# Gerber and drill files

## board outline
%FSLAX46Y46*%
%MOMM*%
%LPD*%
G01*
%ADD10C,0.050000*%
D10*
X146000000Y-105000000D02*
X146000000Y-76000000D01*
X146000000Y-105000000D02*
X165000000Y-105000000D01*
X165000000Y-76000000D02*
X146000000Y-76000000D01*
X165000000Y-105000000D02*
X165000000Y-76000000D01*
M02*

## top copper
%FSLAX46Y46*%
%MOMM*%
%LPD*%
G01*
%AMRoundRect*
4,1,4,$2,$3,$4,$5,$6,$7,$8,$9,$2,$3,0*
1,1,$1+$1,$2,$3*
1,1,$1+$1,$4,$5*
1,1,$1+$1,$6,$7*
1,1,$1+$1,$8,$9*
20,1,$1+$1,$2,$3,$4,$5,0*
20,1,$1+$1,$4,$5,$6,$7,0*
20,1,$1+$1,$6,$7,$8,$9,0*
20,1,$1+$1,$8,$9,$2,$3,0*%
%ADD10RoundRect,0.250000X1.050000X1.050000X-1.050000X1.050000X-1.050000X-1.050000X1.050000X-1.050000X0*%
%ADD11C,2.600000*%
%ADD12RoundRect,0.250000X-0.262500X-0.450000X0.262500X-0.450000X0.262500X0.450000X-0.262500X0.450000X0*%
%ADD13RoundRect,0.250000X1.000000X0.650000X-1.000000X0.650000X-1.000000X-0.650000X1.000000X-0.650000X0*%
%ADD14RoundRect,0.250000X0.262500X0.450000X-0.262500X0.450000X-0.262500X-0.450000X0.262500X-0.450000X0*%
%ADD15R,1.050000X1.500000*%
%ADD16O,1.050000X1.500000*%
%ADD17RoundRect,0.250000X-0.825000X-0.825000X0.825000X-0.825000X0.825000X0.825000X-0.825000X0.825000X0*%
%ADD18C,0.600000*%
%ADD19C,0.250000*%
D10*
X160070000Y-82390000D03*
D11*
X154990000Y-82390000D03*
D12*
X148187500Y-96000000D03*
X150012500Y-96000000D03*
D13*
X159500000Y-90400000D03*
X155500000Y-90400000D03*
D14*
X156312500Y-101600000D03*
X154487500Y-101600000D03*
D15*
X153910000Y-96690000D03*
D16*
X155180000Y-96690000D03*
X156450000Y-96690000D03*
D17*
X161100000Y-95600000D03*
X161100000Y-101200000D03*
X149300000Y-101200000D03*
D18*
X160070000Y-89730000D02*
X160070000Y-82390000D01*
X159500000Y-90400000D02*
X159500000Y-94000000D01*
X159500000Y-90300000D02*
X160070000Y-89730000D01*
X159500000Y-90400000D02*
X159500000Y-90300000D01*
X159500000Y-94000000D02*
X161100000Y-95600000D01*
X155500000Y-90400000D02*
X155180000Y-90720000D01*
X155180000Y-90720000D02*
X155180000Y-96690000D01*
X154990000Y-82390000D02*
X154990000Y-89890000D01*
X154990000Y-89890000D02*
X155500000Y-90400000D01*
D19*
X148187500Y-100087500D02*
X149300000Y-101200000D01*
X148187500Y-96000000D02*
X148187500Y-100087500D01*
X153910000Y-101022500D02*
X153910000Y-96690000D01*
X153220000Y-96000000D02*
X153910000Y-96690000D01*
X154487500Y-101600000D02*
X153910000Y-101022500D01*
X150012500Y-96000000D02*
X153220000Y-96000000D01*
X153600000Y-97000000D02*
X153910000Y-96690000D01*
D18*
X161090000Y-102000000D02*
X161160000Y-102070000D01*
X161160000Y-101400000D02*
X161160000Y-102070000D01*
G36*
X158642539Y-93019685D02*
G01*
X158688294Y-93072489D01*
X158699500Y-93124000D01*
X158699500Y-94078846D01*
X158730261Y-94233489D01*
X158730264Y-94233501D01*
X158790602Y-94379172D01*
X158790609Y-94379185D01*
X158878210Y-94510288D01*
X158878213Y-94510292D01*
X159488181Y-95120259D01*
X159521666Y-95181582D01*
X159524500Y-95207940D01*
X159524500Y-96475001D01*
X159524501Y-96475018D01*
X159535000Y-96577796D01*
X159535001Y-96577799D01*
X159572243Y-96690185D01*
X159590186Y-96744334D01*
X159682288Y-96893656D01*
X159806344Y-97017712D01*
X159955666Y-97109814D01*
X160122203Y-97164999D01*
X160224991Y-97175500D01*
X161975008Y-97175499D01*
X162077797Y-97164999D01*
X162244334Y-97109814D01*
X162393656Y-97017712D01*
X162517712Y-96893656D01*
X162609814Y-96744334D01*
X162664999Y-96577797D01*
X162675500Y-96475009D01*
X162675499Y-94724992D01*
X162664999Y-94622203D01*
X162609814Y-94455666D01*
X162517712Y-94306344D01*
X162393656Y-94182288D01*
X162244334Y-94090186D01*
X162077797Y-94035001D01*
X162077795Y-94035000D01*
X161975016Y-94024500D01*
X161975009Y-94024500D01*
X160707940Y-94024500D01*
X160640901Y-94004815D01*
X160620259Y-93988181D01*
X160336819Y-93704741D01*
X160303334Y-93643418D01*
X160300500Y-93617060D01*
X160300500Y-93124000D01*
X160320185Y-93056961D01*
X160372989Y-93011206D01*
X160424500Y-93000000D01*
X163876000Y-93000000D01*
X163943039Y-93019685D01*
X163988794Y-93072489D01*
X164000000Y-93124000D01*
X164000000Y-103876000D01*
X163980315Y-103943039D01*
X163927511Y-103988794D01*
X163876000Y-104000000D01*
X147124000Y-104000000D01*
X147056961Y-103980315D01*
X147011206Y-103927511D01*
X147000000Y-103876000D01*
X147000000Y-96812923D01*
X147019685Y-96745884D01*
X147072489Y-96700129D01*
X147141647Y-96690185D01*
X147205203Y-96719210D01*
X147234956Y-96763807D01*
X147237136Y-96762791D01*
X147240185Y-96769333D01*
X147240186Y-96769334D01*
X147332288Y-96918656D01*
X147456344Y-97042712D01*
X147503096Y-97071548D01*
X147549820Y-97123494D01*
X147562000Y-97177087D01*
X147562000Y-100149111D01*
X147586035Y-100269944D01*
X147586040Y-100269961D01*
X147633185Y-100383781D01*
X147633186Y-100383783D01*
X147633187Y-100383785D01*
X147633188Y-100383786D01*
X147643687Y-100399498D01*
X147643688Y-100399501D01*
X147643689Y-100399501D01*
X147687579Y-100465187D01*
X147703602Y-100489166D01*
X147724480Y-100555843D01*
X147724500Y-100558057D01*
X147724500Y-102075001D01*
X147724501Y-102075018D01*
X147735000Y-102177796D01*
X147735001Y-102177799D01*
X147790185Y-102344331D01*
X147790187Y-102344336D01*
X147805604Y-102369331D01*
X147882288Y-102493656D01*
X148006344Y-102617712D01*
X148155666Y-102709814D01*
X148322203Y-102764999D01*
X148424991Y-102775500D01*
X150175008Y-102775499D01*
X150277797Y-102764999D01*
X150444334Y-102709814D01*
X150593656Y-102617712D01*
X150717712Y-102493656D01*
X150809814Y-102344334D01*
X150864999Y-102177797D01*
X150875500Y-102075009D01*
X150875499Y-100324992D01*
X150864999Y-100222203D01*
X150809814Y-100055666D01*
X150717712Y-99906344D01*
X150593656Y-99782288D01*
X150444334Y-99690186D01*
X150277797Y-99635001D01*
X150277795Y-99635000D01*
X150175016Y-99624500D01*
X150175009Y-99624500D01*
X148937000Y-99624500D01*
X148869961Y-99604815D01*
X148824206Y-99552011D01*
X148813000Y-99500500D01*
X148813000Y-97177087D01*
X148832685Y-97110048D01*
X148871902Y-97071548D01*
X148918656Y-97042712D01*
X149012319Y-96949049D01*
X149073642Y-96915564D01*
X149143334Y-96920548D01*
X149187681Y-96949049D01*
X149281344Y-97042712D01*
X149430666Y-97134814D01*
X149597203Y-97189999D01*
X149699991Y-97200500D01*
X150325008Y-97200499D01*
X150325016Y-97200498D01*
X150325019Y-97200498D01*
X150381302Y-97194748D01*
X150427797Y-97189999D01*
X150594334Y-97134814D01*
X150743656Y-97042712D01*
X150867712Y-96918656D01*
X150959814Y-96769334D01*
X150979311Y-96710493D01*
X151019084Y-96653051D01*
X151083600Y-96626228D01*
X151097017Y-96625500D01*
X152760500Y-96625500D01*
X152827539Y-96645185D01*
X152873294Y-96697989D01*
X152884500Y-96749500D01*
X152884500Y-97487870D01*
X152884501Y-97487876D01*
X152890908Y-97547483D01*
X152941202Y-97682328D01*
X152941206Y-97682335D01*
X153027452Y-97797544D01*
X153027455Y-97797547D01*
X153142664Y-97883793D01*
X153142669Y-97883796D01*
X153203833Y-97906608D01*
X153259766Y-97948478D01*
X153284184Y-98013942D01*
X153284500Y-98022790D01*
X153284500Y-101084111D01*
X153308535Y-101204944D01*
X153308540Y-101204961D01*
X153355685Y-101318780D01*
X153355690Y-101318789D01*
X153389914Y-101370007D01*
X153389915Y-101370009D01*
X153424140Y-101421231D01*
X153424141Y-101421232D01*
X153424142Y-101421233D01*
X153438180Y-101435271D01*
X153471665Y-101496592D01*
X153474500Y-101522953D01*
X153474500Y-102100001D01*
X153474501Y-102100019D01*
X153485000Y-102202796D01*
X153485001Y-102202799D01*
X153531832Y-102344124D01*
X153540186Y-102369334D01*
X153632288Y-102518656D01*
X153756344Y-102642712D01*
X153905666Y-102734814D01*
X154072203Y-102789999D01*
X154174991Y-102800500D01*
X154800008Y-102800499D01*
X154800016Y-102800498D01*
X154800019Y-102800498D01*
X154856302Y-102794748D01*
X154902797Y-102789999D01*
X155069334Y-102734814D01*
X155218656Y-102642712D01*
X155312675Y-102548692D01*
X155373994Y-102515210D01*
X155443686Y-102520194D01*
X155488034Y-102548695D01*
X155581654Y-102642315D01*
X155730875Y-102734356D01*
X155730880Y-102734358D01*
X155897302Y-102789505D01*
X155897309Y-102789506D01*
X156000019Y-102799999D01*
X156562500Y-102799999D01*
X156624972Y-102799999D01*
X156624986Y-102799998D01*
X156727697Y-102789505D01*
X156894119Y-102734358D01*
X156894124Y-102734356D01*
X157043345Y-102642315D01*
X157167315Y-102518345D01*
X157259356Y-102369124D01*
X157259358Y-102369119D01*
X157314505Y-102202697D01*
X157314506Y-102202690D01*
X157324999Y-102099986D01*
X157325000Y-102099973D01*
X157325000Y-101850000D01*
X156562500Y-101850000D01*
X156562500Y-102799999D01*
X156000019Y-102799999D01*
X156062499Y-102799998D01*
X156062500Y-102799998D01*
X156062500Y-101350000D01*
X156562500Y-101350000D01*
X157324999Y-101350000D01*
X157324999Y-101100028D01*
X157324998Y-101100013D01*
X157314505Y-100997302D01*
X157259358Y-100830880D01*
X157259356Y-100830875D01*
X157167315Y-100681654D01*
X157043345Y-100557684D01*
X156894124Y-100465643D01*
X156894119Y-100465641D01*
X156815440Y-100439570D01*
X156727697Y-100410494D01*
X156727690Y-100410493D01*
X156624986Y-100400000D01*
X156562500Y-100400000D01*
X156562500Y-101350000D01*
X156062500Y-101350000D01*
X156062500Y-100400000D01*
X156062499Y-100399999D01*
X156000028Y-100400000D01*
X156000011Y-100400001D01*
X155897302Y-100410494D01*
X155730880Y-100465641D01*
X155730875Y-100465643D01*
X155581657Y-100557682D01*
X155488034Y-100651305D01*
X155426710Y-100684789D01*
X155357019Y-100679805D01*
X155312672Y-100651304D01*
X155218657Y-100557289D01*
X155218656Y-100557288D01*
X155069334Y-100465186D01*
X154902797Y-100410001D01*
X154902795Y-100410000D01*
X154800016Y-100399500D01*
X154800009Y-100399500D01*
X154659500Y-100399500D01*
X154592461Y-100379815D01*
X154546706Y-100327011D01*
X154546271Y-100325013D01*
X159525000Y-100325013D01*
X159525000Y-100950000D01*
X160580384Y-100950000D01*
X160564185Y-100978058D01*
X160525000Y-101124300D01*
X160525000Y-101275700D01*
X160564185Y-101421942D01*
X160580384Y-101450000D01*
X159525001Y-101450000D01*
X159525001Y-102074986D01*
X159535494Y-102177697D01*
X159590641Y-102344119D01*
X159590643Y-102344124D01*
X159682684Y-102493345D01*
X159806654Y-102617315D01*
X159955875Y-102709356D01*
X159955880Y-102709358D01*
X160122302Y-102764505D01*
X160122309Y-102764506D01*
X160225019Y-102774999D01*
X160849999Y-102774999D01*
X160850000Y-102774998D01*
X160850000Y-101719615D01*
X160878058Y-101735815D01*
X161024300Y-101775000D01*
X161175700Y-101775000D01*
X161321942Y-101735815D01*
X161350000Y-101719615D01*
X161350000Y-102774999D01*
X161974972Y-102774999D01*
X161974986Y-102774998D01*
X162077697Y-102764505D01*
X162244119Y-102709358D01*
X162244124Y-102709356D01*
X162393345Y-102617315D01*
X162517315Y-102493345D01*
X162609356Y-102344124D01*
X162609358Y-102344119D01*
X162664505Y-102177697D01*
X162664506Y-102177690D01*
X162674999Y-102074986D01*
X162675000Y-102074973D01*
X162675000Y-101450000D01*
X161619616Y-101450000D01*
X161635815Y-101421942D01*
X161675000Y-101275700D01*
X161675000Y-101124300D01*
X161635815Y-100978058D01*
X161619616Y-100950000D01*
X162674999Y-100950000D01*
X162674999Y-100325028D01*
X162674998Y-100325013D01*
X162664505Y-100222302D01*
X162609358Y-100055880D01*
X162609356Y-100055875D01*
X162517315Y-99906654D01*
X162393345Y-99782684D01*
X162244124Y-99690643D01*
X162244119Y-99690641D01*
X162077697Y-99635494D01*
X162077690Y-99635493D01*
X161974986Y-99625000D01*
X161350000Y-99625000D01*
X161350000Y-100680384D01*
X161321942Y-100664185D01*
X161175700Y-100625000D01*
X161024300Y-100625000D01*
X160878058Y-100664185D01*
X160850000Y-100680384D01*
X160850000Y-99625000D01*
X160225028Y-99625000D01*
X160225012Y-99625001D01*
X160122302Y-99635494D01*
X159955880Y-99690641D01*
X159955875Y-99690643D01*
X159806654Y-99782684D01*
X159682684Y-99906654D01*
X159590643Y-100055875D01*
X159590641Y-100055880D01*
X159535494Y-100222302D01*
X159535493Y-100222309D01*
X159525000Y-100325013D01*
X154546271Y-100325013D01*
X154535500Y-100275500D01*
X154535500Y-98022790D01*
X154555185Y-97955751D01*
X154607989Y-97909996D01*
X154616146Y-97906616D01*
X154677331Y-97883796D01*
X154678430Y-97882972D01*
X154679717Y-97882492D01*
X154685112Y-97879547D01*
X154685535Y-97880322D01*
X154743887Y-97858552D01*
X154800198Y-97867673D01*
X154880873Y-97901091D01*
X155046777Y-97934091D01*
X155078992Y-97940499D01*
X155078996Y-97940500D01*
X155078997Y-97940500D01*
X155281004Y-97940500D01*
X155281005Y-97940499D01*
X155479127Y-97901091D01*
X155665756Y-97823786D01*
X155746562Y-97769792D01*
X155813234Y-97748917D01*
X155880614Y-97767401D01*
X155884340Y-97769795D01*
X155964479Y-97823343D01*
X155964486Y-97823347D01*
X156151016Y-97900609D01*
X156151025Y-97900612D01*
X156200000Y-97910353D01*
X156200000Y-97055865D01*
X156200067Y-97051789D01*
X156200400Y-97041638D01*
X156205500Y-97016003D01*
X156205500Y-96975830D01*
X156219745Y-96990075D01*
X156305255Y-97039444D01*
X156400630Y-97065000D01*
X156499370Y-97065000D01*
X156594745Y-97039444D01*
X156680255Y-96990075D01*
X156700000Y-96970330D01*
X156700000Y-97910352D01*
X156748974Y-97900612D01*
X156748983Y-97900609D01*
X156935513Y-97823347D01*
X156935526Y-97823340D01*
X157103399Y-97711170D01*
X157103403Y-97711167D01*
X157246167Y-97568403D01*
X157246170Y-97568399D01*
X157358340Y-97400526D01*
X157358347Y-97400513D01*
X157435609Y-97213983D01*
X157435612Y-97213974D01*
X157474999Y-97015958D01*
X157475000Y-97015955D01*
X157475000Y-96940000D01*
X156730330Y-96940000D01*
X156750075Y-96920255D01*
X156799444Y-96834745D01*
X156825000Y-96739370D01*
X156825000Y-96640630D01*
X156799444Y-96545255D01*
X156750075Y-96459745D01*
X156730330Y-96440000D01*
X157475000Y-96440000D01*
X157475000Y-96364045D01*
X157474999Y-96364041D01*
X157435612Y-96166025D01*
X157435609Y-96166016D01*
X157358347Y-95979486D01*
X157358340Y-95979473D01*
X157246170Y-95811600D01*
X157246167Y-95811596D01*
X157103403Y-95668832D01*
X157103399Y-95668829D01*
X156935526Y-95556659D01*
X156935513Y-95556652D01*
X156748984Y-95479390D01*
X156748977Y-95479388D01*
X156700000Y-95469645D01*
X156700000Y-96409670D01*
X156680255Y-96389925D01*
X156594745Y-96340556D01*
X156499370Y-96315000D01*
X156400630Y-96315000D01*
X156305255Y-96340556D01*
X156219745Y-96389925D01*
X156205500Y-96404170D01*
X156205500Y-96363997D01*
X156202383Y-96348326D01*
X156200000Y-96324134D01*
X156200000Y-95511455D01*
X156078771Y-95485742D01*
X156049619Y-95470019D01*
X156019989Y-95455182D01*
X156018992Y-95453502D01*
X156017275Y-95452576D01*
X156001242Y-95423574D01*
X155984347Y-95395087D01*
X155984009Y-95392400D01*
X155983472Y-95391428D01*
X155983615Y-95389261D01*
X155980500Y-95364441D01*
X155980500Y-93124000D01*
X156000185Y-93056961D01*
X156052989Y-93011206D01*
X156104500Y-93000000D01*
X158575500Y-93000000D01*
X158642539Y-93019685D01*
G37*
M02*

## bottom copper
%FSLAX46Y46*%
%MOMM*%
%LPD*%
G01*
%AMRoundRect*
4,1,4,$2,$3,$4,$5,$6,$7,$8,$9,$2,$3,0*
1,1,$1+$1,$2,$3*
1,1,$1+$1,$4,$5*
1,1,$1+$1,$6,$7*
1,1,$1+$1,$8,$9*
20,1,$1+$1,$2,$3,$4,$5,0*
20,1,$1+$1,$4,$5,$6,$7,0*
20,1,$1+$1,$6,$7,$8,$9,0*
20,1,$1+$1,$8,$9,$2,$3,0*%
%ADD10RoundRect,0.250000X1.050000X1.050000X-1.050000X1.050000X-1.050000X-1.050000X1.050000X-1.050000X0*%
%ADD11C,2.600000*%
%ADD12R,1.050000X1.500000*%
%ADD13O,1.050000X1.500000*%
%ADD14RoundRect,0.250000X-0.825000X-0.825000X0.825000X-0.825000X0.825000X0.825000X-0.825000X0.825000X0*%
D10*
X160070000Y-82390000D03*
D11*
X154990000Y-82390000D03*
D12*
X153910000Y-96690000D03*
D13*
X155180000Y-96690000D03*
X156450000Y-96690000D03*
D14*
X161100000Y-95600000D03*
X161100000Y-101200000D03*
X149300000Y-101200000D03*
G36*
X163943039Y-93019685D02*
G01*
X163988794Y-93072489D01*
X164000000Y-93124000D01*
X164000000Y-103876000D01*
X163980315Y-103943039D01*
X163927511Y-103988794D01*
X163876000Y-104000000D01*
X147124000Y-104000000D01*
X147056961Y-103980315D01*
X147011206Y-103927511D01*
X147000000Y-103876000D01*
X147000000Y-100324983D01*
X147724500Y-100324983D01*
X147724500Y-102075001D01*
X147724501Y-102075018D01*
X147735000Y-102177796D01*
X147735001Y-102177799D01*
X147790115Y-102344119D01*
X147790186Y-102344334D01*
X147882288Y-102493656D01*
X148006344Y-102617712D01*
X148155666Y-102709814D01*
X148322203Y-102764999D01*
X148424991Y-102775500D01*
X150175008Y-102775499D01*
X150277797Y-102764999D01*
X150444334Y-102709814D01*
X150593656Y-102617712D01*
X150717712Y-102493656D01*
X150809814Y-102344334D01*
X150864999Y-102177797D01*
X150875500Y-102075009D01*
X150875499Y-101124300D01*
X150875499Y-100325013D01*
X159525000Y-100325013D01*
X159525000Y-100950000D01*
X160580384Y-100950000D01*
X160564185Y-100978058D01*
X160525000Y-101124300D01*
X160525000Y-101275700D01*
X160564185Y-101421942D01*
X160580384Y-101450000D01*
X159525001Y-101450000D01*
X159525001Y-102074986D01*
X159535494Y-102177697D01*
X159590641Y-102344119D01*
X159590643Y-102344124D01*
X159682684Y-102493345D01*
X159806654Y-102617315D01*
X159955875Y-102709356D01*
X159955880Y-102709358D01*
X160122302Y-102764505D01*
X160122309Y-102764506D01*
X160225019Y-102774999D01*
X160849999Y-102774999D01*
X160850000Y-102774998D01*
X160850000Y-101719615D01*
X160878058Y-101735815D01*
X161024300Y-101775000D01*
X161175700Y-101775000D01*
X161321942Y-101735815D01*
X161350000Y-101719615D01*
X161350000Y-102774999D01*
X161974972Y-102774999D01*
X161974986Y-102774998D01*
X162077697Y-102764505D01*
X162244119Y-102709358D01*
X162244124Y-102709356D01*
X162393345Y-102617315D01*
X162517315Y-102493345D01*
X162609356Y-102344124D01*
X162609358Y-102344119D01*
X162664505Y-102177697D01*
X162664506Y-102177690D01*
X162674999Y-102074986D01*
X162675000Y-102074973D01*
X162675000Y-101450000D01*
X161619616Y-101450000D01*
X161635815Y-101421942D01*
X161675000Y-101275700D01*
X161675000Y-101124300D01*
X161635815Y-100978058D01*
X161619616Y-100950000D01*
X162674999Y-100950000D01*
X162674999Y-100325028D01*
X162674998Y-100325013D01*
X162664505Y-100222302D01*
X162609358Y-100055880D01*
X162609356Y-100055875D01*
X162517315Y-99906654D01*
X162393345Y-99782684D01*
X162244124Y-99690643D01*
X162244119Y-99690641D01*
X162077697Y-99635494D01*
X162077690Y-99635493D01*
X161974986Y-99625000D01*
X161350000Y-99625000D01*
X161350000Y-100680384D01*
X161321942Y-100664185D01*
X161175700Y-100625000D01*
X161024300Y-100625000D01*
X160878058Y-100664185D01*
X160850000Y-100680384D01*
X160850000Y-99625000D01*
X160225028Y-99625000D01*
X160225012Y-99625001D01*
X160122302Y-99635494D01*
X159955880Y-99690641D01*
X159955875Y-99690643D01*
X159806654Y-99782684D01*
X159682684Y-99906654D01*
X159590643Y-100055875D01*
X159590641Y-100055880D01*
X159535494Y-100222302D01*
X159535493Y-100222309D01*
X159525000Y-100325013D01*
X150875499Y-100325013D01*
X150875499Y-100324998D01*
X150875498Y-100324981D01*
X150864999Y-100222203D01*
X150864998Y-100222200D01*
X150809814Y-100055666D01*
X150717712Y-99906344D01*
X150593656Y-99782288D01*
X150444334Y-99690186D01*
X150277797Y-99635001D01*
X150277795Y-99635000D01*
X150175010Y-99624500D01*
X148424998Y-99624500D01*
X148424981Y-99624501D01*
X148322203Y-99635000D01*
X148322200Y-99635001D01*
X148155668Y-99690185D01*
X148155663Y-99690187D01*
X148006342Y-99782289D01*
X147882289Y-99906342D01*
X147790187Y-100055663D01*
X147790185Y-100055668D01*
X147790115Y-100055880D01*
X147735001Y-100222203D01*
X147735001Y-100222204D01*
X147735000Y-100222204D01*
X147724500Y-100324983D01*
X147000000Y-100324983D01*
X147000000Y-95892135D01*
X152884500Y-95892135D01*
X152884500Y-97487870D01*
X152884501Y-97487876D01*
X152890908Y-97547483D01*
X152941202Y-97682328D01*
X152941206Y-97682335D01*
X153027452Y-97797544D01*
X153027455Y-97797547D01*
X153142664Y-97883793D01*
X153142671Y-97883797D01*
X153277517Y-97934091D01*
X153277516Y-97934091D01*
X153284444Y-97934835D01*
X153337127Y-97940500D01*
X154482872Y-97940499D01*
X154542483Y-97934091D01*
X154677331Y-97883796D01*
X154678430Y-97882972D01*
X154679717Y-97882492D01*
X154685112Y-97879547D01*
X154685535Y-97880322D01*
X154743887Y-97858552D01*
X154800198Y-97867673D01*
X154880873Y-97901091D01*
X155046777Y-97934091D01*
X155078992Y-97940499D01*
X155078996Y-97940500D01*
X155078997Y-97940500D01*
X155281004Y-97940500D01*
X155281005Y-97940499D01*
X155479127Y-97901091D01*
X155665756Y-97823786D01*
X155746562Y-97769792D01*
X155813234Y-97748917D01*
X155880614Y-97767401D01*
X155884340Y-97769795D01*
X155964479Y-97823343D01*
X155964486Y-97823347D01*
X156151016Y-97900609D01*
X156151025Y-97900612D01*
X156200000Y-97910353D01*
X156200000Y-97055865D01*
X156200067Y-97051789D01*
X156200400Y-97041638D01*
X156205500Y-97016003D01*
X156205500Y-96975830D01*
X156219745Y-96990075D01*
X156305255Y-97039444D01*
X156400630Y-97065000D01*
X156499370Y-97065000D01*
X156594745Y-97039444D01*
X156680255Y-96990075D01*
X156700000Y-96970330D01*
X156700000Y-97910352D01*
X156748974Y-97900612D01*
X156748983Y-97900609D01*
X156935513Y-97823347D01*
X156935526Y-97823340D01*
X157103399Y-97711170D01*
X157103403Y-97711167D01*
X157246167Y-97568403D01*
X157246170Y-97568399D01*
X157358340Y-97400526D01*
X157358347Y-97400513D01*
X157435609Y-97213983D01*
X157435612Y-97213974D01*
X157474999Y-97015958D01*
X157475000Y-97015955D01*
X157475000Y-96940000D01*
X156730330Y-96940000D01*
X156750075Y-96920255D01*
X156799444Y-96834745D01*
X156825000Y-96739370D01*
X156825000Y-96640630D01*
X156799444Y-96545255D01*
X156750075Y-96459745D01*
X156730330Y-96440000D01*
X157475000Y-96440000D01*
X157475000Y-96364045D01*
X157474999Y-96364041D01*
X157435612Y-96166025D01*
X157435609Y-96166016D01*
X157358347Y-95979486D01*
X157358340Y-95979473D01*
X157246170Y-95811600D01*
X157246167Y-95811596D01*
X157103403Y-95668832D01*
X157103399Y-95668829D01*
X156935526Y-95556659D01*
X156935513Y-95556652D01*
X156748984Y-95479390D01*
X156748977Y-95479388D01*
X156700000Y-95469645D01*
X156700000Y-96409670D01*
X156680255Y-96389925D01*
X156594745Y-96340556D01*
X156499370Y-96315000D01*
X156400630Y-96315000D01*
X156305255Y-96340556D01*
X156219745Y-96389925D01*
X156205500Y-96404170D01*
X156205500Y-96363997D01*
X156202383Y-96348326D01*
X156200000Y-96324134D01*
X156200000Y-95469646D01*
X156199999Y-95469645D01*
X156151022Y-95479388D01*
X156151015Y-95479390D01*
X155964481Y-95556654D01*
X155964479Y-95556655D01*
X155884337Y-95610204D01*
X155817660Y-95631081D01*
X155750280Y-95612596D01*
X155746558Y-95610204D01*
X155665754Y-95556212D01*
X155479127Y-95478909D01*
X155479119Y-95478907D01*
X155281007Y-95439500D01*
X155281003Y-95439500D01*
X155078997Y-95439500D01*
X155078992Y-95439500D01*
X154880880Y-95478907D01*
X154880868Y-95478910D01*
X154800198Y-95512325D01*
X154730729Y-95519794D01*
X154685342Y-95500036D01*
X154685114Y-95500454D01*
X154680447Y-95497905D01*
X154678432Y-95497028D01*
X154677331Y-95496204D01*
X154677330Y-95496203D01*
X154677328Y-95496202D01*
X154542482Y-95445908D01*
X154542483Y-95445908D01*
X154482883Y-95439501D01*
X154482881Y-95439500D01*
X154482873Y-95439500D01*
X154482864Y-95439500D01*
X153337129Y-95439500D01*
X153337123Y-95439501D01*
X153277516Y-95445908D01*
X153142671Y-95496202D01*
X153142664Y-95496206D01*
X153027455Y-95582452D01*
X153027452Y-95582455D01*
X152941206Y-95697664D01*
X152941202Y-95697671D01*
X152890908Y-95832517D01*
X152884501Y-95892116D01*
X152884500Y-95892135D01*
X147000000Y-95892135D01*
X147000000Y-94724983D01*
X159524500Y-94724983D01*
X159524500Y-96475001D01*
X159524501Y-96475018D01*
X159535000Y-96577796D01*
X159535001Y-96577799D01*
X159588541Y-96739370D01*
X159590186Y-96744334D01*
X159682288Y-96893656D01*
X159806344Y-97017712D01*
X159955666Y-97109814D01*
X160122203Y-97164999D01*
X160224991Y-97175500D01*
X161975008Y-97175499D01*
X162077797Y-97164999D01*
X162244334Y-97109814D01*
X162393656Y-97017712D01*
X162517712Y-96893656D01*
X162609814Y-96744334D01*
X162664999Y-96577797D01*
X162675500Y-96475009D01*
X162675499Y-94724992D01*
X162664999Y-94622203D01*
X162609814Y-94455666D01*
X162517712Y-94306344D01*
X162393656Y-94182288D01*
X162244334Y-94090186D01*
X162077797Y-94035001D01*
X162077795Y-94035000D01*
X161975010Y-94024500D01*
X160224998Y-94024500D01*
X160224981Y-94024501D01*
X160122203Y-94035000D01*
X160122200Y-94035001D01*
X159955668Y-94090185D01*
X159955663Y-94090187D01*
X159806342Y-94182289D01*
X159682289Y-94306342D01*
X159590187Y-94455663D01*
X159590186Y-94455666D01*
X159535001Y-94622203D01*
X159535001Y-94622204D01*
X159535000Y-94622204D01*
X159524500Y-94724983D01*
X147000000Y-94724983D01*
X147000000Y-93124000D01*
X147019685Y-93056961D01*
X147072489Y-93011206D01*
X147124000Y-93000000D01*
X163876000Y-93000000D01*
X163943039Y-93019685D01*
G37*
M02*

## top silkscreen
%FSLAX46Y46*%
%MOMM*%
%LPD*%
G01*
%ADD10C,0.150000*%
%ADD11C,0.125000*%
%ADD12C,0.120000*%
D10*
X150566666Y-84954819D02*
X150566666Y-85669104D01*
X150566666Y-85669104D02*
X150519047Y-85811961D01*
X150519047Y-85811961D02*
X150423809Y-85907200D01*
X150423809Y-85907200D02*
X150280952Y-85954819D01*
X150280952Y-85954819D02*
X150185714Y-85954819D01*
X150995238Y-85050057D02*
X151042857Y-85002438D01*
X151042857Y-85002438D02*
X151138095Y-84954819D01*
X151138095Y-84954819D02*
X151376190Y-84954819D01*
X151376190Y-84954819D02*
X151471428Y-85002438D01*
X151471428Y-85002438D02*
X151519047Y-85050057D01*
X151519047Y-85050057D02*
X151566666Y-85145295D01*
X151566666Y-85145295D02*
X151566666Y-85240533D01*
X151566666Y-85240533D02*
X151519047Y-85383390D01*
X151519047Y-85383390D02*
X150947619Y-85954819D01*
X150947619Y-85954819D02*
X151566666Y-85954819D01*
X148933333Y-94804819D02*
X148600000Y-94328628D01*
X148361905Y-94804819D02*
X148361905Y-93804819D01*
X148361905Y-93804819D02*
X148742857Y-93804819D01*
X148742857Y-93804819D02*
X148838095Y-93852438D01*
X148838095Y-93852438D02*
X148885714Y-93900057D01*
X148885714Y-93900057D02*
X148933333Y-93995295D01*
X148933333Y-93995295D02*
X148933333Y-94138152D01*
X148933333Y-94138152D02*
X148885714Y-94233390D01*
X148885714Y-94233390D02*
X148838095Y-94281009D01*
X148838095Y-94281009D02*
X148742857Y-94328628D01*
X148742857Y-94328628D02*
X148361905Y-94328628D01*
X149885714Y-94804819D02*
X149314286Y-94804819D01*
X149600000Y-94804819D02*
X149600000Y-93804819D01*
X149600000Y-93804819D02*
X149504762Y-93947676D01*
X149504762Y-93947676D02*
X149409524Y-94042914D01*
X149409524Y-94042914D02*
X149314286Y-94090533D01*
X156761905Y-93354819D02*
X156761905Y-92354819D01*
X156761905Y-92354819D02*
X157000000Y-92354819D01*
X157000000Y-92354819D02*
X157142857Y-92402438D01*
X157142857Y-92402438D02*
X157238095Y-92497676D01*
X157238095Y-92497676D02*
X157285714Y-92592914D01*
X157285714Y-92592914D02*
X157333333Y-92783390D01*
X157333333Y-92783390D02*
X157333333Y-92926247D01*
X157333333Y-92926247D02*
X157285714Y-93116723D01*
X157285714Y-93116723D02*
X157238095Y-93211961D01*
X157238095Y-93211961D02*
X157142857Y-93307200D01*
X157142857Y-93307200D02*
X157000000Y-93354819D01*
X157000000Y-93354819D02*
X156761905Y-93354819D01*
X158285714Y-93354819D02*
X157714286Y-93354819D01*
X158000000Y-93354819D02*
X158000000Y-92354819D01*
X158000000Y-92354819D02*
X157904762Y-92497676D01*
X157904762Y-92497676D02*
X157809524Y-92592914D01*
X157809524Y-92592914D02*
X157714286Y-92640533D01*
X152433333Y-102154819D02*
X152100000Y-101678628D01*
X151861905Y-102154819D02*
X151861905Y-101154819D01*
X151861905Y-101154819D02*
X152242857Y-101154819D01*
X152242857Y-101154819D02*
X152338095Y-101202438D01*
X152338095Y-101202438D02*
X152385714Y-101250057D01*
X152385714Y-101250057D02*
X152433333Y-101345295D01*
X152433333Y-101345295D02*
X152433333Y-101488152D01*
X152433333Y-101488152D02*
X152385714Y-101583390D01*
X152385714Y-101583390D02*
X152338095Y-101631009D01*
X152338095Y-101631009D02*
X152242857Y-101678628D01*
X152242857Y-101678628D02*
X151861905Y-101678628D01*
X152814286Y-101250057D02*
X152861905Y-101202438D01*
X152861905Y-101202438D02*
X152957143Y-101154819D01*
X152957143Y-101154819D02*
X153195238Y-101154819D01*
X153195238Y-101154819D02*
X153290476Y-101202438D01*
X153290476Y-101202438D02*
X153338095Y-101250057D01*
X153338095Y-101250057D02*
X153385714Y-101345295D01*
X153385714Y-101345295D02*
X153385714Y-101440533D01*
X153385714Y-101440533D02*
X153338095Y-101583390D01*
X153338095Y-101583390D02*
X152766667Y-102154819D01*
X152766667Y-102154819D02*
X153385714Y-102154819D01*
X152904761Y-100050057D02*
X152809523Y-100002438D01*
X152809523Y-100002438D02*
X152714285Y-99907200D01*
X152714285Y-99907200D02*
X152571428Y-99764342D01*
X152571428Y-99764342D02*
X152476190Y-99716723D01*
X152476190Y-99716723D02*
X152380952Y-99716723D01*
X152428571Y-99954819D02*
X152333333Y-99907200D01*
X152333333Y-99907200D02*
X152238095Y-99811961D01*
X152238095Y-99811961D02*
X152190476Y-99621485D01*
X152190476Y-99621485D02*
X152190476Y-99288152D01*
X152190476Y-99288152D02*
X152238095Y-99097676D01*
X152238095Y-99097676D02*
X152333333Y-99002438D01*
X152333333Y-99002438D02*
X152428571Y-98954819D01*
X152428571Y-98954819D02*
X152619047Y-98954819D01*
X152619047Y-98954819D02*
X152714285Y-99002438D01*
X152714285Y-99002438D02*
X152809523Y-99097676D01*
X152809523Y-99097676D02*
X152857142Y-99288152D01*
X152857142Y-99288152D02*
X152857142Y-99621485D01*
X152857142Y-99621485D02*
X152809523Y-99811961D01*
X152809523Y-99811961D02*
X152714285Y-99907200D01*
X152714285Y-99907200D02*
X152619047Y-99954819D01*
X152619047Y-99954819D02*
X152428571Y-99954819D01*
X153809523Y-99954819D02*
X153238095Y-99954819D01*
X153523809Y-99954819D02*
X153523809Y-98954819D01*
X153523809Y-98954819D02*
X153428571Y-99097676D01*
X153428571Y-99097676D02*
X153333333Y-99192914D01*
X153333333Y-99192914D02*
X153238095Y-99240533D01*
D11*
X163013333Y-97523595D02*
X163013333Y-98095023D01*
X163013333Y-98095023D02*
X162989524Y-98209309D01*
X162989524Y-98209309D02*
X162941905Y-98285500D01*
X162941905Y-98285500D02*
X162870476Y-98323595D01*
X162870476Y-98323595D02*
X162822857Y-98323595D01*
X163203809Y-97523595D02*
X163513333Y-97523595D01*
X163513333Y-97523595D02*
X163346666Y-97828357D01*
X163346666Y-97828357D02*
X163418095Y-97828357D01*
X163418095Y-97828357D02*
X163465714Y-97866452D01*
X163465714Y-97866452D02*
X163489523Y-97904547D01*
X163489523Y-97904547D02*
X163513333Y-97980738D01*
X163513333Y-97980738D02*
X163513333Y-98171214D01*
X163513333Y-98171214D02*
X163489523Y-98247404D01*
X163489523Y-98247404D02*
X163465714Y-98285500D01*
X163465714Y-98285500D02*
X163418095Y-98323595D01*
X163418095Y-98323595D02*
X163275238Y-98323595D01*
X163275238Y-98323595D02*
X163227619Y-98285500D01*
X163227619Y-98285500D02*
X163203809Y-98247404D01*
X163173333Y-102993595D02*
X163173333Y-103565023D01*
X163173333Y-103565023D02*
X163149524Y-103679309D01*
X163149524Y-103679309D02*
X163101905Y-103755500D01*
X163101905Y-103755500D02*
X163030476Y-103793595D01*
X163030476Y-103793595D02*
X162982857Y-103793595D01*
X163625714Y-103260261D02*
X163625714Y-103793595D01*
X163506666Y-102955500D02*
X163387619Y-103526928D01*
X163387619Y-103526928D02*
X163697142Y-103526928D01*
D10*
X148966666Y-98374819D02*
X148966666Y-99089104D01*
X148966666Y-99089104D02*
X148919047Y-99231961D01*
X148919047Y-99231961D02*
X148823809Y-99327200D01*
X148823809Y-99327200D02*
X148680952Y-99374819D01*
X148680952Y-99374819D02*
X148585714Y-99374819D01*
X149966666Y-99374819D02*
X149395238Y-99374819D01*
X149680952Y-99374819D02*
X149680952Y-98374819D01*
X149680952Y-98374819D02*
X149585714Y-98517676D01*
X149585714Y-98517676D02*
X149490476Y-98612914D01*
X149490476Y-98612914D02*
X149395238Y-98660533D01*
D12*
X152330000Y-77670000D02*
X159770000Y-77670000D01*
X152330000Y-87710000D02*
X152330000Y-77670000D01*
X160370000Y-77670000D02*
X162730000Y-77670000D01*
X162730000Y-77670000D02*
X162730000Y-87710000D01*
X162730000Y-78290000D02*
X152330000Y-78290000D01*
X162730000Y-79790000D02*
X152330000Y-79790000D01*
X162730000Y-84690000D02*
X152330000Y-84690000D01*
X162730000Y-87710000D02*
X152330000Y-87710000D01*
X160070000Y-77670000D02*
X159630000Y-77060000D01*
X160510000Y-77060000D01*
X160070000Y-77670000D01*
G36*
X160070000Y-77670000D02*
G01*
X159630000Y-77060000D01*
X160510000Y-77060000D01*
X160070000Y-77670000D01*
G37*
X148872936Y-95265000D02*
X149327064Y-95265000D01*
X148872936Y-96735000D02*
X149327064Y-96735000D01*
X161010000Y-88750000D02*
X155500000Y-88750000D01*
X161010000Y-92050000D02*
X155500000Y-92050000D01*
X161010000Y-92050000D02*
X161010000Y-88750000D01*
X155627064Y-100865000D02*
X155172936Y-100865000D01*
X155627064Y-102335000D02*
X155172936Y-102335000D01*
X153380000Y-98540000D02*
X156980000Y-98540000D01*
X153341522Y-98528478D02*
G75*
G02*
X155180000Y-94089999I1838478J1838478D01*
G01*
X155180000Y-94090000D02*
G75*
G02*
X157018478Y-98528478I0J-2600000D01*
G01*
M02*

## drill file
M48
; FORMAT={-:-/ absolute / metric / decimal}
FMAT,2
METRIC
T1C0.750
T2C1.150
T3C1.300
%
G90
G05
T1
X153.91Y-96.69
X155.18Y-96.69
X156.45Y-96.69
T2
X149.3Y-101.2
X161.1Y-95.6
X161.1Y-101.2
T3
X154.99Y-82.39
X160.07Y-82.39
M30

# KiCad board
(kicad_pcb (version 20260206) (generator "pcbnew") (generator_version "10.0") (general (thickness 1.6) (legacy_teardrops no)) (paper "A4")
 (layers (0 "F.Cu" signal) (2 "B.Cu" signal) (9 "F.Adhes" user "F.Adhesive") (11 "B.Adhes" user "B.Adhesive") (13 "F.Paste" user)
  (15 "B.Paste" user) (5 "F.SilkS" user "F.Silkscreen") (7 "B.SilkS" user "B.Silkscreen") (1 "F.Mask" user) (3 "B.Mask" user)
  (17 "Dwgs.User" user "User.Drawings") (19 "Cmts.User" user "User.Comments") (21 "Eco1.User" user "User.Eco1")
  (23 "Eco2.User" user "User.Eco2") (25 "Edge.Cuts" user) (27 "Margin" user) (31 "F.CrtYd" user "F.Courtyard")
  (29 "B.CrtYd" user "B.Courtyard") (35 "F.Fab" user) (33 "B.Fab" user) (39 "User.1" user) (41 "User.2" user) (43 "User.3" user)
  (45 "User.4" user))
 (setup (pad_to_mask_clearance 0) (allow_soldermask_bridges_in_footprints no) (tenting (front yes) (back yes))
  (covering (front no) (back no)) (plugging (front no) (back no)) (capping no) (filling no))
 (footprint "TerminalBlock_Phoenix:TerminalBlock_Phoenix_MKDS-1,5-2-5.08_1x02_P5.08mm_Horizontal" (layer "F.Cu") (at 160.07 82.39 180)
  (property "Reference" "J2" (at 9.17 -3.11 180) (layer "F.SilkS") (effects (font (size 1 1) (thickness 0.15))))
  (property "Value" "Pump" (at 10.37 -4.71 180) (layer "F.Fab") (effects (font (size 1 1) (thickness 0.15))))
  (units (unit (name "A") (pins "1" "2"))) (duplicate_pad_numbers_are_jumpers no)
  (fp_line (start 7.74 4.72) (end 0.3 4.72) (stroke (width 0.12) (type solid)) (layer "F.SilkS"))
  (fp_line (start 7.74 -5.32) (end 7.74 4.72) (stroke (width 0.12) (type solid)) (layer "F.SilkS"))
  (fp_line (start -0.3 4.72) (end -2.66 4.72) (stroke (width 0.12) (type solid)) (layer "F.SilkS"))
  (fp_line (start -2.66 4.72) (end -2.66 -5.32) (stroke (width 0.12) (type solid)) (layer "F.SilkS"))
  (fp_line (start -2.66 4.1) (end 7.74 4.1) (stroke (width 0.12) (type solid)) (layer "F.SilkS"))
  (fp_line (start -2.66 2.6) (end 7.74 2.6) (stroke (width 0.12) (type solid)) (layer "F.SilkS"))
  (fp_line (start -2.66 -2.3) (end 7.74 -2.3) (stroke (width 0.12) (type solid)) (layer "F.SilkS"))
  (fp_line (start -2.66 -5.32) (end 7.74 -5.32) (stroke (width 0.12) (type solid)) (layer "F.SilkS"))
  (fp_poly (pts (xy 0 4.72) (xy 0.44 5.33) (xy -0.44 5.33)) (stroke (width 0.12) (type solid)) (fill yes) (layer "F.SilkS"))
  (pad "1" thru_hole roundrect (at 0 0 180) (size 2.6 2.6) (drill 1.3) (layers "*.Cu" "*.Mask") (remove_unused_layers no)
   (roundrect_rratio 0.096154) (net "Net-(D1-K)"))
  (pad "2" thru_hole circle (at 5.08 0 180) (size 2.6 2.6) (drill 1.3) (layers "*.Cu" "*.Mask") (remove_unused_layers no) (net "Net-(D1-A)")))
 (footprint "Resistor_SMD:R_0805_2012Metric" (layer "F.Cu") (at 149.1 96)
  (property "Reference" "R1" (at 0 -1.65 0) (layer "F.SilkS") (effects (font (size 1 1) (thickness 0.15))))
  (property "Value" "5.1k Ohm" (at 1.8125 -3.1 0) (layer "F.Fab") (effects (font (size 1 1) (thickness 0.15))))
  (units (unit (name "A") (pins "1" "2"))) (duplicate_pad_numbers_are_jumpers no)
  (fp_line (start -0.227064 -0.735) (end 0.227064 -0.735) (stroke (width 0.12) (type solid)) (layer "F.SilkS"))
  (fp_line (start -0.227064 0.735) (end 0.227064 0.735) (stroke (width 0.12) (type solid)) (layer "F.SilkS"))
  (pad "1" smd roundrect (at -0.9125 0) (size 1.025 1.4) (layers "F.Cu" "F.Mask" "F.Paste") (roundrect_rratio 0.243902)
   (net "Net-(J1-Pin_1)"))
  (pad "2" smd roundrect (at 0.9125 0) (size 1.025 1.4) (layers "F.Cu" "F.Mask" "F.Paste") (roundrect_rratio 0.243902) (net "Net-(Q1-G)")))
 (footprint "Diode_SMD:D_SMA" (layer "F.Cu") (at 157.5 90.4 180)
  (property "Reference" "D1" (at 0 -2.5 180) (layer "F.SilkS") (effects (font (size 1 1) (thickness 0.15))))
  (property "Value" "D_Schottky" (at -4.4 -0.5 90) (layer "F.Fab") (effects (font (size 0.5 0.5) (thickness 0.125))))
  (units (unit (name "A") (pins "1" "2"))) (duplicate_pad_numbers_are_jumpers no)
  (fp_line (start -3.51 1.65) (end 2 1.65) (stroke (width 0.12) (type solid)) (layer "F.SilkS"))
  (fp_line (start -3.51 -1.65) (end 2 -1.65) (stroke (width 0.12) (type solid)) (layer "F.SilkS"))
  (fp_line (start -3.51 -1.65) (end -3.51 1.65) (stroke (width 0.12) (type solid)) (layer "F.SilkS"))
  (pad "1" smd roundrect (at -2 0 180) (size 2.5 1.8) (layers "F.Cu" "F.Mask" "F.Paste") (roundrect_rratio 0.1388888889) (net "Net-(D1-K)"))
  (pad "2" smd roundrect (at 2 0 180) (size 2.5 1.8) (layers "F.Cu" "F.Mask" "F.Paste") (roundrect_rratio 0.1388888889) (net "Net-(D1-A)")))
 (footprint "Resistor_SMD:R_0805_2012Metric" (layer "F.Cu") (at 155.4 101.6 180)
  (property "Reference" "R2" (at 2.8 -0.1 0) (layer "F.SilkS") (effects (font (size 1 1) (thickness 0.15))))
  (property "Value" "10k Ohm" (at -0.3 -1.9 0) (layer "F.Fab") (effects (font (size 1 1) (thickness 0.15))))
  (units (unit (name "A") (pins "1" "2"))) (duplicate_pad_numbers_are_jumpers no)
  (fp_line (start -0.227064 0.735) (end 0.227064 0.735) (stroke (width 0.12) (type solid)) (layer "F.SilkS"))
  (fp_line (start -0.227064 -0.735) (end 0.227064 -0.735) (stroke (width 0.12) (type solid)) (layer "F.SilkS"))
  (pad "1" smd roundrect (at -0.9125 0 180) (size 1.025 1.4) (layers "F.Cu" "F.Mask" "F.Paste") (roundrect_rratio 0.243902) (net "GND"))
  (pad "2" smd roundrect (at 0.9125 0 180) (size 1.025 1.4) (layers "F.Cu" "F.Mask" "F.Paste") (roundrect_rratio 0.243902)
   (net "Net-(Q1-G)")))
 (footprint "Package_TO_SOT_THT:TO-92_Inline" (layer "F.Cu") (at 153.91 96.69)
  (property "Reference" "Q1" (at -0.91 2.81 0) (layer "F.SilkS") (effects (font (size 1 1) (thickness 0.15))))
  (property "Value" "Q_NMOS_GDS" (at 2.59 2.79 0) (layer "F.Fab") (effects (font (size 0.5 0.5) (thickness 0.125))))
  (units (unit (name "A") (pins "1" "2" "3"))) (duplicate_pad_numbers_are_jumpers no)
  (fp_line (start -0.53 1.85) (end 3.07 1.85) (stroke (width 0.12) (type solid)) (layer "F.SilkS"))
  (fp_arc (start -0.568478 1.838478) (mid -1.132087 -0.994977) (end 1.27 -2.6) (stroke (width 0.12) (type solid)) (layer "F.SilkS"))
  (fp_arc (start 1.27 -2.6) (mid 3.672087 -0.994977) (end 3.108478 1.838478) (stroke (width 0.12) (type solid)) (layer "F.SilkS"))
  (pad "1" thru_hole rect (at 0 0) (size 1.05 1.5) (drill 0.75) (layers "*.Cu" "*.Mask") (remove_unused_layers no) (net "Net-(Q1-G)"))
  (pad "2" thru_hole oval (at 1.27 0) (size 1.05 1.5) (drill 0.75) (layers "*.Cu" "*.Mask") (remove_unused_layers no) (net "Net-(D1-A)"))
  (pad "3" thru_hole oval (at 2.54 0) (size 1.05 1.5) (drill 0.75) (layers "*.Cu" "*.Mask") (remove_unused_layers no) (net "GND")))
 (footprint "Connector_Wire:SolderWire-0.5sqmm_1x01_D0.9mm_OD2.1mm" (layer "F.Cu") (at 161.1 95.6)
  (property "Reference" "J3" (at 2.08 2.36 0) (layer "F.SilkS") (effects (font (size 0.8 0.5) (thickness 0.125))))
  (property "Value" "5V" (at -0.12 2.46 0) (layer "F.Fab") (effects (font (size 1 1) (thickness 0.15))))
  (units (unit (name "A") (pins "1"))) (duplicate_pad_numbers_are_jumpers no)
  (pad "1" thru_hole roundrect (at 0 0) (size 2.15 2.15) (drill 1.15) (layers "*.Cu" "*.Mask") (remove_unused_layers no)
   (roundrect_rratio 0.116279) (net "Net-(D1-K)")))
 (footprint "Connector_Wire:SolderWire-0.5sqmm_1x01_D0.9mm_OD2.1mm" (layer "F.Cu") (at 161.1 101.2)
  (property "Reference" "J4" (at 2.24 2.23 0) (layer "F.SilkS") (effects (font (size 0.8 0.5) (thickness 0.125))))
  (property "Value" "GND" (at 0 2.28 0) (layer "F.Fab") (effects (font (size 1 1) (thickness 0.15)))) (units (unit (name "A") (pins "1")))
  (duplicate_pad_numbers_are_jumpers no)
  (pad "1" thru_hole roundrect (at 0 0) (size 2.15 2.15) (drill 1.15) (layers "*.Cu" "*.Mask") (remove_unused_layers no)
   (roundrect_rratio 0.116279) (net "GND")))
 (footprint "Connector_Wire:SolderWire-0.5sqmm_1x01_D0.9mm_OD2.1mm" (layer "F.Cu") (at 149.3 101.2)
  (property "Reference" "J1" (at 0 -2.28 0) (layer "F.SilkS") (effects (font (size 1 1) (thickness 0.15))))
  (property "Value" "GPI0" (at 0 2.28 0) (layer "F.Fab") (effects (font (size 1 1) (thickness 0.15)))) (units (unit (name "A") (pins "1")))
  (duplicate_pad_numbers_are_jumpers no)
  (pad "1" thru_hole roundrect (at 0 0) (size 2.15 2.15) (drill 1.15) (layers "*.Cu" "*.Mask") (remove_unused_layers no)
   (roundrect_rratio 0.116279) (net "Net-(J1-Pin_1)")))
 (gr_line (start 146 105) (end 146 76) (stroke (width 0.05) (type default)) (layer "Edge.Cuts"))
 (gr_line (start 146 105) (end 165 105) (stroke (width 0.05) (type default)) (layer "Edge.Cuts"))
 (gr_line (start 165 76) (end 146 76) (stroke (width 0.05) (type default)) (layer "Edge.Cuts"))
 (gr_line (start 165 105) (end 165 76) (stroke (width 0.05) (type default)) (layer "Edge.Cuts"))
 (segment (start 160.07 89.73) (end 160.07 82.39) (width 0.6) (layer "F.Cu") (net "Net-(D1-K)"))
 (segment (start 159.5 90.4) (end 159.5 94) (width 0.6) (layer "F.Cu") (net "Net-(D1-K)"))
 (segment (start 159.5 90.3) (end 160.07 89.73) (width 0.6) (layer "F.Cu") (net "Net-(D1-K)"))
 (segment (start 159.5 90.4) (end 159.5 90.3) (width 0.6) (layer "F.Cu") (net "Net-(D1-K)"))
 (segment (start 159.5 94) (end 161.1 95.6) (width 0.6) (layer "F.Cu") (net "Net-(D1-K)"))
 (segment (start 155.5 90.4) (end 155.18 90.72) (width 0.6) (layer "F.Cu") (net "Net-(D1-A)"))
 (segment (start 155.18 90.72) (end 155.18 96.69) (width 0.6) (layer "F.Cu") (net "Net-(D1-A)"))
 (segment (start 154.99 82.39) (end 154.99 89.89) (width 0.6) (layer "F.Cu") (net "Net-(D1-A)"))
 (segment (start 154.99 89.89) (end 155.5 90.4) (width 0.6) (layer "F.Cu") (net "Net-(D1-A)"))
 (segment (start 148.1875 100.0875) (end 149.3 101.2) (width 0.25) (layer "F.Cu") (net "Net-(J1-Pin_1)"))
 (segment (start 148.1875 96) (end 148.1875 100.0875) (width 0.25) (layer "F.Cu") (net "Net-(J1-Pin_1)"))
 (segment (start 153.91 101.0225) (end 153.91 96.69) (width 0.25) (layer "F.Cu") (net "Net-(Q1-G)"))
 (segment (start 153.22 96) (end 153.91 96.69) (width 0.25) (layer "F.Cu") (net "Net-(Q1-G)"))
 (segment (start 154.4875 101.6) (end 153.91 101.0225) (width 0.25) (layer "F.Cu") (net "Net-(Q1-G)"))
 (segment (start 150.0125 96) (end 153.22 96) (width 0.25) (layer "F.Cu") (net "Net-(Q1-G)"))
 (segment (start 153.6 97) (end 153.91 96.69) (width 0.25) (layer "F.Cu") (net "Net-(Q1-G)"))
 (segment (start 161.09 102) (end 161.16 102.07) (width 0.6) (layer "F.Cu") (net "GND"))
 (segment (start 161.16 101.4) (end 161.16 102.07) (width 0.6) (layer "F.Cu") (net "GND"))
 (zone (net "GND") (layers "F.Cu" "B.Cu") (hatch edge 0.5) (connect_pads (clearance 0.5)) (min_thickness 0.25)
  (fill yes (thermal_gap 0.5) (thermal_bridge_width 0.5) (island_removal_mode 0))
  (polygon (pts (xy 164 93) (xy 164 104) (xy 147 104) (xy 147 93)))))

